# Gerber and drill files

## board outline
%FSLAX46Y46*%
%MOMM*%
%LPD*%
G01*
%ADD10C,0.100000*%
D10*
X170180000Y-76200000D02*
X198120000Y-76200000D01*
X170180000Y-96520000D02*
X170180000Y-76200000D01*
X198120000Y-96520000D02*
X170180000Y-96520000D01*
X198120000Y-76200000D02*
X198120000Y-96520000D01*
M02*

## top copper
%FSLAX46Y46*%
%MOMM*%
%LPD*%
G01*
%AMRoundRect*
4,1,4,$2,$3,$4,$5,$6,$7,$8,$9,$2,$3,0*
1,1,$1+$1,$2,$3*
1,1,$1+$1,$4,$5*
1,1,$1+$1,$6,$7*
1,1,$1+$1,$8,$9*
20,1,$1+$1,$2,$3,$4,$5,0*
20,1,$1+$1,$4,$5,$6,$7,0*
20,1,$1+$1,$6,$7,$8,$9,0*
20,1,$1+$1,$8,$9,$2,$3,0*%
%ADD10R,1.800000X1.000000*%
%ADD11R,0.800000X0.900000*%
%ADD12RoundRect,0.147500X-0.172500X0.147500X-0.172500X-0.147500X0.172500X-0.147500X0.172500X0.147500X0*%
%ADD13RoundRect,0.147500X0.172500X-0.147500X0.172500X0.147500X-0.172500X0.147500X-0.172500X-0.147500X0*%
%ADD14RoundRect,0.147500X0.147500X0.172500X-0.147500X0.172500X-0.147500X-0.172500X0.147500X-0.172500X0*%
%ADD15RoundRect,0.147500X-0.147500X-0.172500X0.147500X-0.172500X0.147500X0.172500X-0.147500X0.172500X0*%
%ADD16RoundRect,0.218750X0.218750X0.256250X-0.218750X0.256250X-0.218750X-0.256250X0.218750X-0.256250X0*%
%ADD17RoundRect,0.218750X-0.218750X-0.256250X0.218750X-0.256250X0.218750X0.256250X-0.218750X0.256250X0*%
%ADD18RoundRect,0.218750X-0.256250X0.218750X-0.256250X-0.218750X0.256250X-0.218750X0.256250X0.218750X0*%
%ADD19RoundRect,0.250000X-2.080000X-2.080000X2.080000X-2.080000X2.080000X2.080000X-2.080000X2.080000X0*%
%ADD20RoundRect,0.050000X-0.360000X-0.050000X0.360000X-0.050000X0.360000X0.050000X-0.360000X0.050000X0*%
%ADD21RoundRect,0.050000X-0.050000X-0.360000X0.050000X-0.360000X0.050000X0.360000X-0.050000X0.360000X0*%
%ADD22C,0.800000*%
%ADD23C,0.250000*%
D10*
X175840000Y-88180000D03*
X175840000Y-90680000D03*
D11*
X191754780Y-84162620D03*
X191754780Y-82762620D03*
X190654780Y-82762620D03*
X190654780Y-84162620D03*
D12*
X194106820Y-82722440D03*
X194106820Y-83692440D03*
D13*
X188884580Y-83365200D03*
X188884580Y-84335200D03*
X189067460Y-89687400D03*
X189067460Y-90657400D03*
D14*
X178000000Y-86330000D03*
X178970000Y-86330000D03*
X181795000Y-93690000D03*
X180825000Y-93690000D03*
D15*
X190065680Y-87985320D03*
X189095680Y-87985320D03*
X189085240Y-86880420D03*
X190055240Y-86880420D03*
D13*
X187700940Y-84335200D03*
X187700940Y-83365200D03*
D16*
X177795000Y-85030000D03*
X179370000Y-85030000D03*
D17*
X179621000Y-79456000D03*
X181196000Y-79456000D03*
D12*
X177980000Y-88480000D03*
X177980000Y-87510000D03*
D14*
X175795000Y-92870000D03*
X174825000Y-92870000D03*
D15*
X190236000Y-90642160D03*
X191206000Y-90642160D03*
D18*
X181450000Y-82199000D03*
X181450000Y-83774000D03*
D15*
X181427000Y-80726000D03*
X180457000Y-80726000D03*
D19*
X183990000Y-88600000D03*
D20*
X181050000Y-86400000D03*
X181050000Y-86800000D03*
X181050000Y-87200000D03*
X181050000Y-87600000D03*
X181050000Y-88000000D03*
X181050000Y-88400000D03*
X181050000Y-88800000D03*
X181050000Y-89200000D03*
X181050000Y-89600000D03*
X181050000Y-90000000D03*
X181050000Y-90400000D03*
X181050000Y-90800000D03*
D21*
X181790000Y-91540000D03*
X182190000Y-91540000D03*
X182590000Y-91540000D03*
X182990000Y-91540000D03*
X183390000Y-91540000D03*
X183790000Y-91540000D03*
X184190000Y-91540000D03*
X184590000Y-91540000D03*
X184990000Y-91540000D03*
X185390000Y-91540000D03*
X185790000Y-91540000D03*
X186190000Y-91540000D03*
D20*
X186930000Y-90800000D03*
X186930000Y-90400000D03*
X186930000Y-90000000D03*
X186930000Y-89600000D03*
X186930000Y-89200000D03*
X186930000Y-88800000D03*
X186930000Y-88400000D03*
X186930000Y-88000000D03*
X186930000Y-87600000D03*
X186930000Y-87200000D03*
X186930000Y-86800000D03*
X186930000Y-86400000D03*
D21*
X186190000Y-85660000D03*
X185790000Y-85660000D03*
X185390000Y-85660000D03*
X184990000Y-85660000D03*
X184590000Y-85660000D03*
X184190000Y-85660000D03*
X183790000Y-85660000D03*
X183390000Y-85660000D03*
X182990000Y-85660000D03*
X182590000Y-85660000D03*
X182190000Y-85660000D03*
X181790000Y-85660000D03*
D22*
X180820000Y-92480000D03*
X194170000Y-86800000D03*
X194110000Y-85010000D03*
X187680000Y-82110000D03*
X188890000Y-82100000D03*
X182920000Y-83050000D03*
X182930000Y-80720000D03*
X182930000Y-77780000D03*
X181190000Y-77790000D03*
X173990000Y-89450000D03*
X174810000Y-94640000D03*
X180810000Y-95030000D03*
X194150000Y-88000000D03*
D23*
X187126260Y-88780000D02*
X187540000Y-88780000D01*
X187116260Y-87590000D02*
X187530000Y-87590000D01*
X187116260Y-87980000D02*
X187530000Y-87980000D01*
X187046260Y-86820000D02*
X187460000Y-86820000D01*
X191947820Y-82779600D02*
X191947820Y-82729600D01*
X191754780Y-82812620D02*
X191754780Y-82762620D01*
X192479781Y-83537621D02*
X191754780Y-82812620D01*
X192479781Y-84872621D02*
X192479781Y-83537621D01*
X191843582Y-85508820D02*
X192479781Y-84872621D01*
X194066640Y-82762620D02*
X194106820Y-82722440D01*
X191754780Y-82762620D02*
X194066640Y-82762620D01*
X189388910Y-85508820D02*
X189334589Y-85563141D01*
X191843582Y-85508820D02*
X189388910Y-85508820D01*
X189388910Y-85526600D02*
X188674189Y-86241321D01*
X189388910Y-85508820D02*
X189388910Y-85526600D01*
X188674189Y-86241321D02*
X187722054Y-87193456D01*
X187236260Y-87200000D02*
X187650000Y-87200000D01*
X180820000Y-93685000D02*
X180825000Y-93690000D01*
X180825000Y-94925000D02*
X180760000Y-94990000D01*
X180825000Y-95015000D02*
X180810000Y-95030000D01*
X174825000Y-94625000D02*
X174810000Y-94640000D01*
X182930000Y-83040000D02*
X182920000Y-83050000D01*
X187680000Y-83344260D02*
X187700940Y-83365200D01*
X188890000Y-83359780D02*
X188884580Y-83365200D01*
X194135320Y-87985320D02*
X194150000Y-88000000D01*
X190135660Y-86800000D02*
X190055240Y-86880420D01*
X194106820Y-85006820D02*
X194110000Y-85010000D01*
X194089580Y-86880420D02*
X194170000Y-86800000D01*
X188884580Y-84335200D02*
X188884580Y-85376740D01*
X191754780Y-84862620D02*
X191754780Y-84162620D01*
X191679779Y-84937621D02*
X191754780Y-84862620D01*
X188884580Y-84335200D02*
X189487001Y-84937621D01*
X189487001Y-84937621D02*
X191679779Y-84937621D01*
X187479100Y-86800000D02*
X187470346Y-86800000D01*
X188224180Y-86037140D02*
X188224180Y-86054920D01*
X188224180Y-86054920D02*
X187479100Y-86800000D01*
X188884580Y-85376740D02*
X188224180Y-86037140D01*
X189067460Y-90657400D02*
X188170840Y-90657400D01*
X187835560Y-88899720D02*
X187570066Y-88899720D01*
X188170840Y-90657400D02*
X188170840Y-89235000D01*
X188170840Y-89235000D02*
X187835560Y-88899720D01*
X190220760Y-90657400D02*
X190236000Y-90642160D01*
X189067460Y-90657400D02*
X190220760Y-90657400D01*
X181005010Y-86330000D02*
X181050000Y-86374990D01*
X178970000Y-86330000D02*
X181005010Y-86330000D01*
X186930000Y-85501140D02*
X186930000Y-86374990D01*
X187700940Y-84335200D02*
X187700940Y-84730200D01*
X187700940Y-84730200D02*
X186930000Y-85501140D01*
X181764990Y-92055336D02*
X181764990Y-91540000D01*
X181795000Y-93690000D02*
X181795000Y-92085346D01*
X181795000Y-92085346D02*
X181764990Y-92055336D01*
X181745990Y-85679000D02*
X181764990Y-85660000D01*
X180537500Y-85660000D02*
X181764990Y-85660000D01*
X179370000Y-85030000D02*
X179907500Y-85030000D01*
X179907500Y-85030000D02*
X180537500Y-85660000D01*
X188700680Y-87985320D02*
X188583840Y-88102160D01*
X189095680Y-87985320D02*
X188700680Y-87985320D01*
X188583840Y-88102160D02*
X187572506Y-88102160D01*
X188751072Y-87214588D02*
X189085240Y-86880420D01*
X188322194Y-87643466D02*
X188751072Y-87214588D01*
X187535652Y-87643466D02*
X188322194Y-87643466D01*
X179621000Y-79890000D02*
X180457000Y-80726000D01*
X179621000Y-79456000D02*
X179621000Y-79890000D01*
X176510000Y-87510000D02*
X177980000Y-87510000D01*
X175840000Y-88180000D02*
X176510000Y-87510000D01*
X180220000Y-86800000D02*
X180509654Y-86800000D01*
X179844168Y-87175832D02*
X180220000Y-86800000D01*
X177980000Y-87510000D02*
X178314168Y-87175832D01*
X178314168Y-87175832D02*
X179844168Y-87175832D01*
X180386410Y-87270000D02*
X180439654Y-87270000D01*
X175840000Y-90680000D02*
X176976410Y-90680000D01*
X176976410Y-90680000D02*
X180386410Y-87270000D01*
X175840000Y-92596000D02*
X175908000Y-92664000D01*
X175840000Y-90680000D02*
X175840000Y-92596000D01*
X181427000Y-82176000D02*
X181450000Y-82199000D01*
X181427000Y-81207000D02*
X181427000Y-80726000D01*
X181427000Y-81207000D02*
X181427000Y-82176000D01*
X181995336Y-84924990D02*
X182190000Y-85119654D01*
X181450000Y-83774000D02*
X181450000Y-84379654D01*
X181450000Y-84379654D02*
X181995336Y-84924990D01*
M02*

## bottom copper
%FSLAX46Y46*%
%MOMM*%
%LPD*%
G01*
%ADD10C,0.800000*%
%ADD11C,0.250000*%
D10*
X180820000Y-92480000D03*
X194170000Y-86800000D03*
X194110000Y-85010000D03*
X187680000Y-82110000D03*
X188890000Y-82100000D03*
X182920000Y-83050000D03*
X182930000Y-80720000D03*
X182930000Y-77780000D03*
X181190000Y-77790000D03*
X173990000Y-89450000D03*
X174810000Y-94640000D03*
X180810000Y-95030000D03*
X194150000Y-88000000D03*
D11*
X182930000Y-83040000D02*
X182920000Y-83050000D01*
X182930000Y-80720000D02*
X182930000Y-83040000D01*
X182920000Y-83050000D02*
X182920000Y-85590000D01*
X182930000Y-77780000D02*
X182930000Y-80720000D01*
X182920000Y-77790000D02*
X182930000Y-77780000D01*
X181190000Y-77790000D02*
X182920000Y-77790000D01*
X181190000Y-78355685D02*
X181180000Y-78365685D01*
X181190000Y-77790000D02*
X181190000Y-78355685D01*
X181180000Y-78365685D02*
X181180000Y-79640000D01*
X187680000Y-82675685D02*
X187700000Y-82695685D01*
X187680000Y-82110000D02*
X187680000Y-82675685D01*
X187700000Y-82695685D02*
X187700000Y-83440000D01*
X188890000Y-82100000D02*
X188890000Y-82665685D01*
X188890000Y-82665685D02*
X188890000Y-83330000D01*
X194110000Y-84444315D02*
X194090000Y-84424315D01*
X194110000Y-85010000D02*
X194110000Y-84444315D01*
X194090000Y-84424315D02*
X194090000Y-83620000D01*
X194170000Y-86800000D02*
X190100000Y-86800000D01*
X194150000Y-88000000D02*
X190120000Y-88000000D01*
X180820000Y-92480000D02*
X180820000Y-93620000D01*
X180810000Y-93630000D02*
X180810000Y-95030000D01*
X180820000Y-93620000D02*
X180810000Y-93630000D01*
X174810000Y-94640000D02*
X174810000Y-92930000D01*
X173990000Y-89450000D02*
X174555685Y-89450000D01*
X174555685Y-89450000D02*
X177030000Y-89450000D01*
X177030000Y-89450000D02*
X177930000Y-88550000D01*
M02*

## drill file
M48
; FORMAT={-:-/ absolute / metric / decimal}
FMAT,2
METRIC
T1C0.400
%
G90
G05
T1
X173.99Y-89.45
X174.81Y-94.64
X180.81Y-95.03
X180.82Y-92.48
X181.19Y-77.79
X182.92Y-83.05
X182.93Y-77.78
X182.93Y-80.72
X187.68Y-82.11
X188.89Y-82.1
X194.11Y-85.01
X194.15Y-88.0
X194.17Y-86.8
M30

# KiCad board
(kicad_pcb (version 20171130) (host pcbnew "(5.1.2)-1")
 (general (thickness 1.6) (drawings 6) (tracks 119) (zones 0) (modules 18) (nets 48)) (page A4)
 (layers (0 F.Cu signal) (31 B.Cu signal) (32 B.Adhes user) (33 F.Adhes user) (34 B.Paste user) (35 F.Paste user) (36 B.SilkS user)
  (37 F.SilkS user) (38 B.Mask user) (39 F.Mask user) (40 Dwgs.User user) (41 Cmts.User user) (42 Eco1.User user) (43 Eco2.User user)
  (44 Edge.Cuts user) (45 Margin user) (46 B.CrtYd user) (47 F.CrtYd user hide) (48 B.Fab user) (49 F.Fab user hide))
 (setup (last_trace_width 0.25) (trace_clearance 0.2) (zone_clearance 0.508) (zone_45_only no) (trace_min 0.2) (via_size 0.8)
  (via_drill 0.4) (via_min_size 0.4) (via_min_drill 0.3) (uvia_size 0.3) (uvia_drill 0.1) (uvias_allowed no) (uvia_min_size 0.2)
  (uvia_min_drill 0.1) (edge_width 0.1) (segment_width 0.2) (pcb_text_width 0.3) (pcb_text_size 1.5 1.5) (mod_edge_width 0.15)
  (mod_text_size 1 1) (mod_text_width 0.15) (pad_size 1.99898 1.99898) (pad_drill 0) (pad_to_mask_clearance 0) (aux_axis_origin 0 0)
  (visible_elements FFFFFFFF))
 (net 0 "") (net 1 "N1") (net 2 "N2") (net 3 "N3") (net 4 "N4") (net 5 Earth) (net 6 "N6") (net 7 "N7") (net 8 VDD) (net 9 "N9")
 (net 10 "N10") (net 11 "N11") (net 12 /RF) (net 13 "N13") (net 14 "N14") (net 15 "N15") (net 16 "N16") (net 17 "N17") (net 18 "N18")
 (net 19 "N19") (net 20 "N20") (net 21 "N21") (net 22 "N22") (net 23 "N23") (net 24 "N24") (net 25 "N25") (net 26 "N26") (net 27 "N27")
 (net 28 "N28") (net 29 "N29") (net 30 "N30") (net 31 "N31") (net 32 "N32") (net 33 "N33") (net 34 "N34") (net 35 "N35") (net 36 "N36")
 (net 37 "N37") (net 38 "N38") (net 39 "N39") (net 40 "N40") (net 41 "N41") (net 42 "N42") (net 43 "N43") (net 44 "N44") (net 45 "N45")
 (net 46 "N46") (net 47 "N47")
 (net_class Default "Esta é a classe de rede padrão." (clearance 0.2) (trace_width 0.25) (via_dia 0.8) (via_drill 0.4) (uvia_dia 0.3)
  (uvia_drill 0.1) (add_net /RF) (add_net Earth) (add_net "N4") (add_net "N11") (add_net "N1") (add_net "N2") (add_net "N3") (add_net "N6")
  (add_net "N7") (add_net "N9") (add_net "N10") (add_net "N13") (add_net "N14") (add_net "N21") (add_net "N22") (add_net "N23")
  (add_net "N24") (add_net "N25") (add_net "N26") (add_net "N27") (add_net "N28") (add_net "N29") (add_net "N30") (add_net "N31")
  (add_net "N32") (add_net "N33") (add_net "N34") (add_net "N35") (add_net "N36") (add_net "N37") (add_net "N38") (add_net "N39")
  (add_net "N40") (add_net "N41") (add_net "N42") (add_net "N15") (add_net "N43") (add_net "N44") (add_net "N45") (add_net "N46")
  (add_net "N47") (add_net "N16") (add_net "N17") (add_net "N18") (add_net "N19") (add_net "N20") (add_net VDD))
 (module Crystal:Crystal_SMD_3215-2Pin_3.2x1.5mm (layer F.Cu) (at 175.84 89.43 90)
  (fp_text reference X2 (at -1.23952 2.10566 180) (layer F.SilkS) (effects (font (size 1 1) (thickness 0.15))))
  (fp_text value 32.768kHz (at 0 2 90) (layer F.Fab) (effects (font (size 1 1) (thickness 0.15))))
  (pad 1 smd rect (at 1.25 0 90) (size 1 1.8) (layers F.Cu F.Paste F.Mask) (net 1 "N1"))
  (pad 2 smd rect (at -1.25 0 90) (size 1 1.8) (layers F.Cu F.Paste F.Mask) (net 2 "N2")))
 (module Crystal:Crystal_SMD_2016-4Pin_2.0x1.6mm (layer F.Cu) (at 191.20478 83.46262 90)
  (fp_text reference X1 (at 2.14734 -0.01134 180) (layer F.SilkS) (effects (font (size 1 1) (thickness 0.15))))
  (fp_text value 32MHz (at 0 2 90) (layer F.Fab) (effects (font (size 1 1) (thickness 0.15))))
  (pad 1 smd rect (at -0.7 0.55 90) (size 0.9 0.8) (layers F.Cu F.Paste F.Mask) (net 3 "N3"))
  (pad 2 smd rect (at 0.7 0.55 90) (size 0.9 0.8) (layers F.Cu F.Paste F.Mask) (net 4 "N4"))
  (pad 3 smd rect (at 0.7 -0.55 90) (size 0.9 0.8) (layers F.Cu F.Paste F.Mask))
  (pad 4 smd rect (at -0.7 -0.55 90) (size 0.9 0.8) (layers F.Cu F.Paste F.Mask)))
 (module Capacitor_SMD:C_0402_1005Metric (layer F.Cu) (at 194.10682 83.20744 270)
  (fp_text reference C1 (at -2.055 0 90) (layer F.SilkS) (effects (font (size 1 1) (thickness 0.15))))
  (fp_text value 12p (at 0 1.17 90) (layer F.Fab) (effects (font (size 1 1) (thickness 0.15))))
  (pad 1 smd roundrect (at -0.485 0 270) (size 0.59 0.64) (layers F.Cu F.Paste F.Mask) (roundrect_rratio 0.25) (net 4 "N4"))
  (pad 2 smd roundrect (at 0.485 0 270) (size 0.59 0.64) (layers F.Cu F.Paste F.Mask) (roundrect_rratio 0.25) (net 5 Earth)))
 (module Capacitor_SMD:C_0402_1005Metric (layer F.Cu) (at 188.88458 83.8502 90)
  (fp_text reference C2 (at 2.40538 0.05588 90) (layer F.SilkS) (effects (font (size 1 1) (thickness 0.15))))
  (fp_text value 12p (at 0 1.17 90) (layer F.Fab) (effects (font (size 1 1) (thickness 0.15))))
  (pad 2 smd roundrect (at 0.485 0 90) (size 0.59 0.64) (layers F.Cu F.Paste F.Mask) (roundrect_rratio 0.25) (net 5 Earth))
  (pad 1 smd roundrect (at -0.485 0 90) (size 0.59 0.64) (layers F.Cu F.Paste F.Mask) (roundrect_rratio 0.25) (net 3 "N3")))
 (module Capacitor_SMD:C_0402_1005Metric (layer F.Cu) (at 189.06746 90.1724 90)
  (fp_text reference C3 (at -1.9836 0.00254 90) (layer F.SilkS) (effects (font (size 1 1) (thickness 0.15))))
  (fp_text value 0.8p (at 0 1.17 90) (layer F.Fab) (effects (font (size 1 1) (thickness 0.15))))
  (pad 2 smd roundrect (at 0.485 0 90) (size 0.59 0.64) (layers F.Cu F.Paste F.Mask) (roundrect_rratio 0.25) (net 5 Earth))
  (pad 1 smd roundrect (at -0.485 0 90) (size 0.59 0.64) (layers F.Cu F.Paste F.Mask) (roundrect_rratio 0.25) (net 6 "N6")))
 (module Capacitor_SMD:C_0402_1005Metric (layer F.Cu) (at 178.485 86.33 180)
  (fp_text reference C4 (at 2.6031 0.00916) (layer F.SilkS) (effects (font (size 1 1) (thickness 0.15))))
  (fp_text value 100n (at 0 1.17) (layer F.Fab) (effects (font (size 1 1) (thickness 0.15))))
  (pad 2 smd roundrect (at 0.485 0 180) (size 0.59 0.64) (layers F.Cu F.Paste F.Mask) (roundrect_rratio 0.25) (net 5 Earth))
  (pad 1 smd roundrect (at -0.485 0 180) (size 0.59 0.64) (layers F.Cu F.Paste F.Mask) (roundrect_rratio 0.25) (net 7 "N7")))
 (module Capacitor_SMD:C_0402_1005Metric (layer F.Cu) (at 181.31 93.69 180)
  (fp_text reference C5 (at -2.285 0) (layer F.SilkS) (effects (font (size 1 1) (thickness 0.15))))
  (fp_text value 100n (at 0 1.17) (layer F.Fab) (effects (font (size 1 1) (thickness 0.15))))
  (pad 1 smd roundrect (at -0.485 0 180) (size 0.59 0.64) (layers F.Cu F.Paste F.Mask) (roundrect_rratio 0.25) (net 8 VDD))
  (pad 2 smd roundrect (at 0.485 0 180) (size 0.59 0.64) (layers F.Cu F.Paste F.Mask) (roundrect_rratio 0.25) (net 5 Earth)))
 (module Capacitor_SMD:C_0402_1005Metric (layer F.Cu) (at 189.58068 87.98532)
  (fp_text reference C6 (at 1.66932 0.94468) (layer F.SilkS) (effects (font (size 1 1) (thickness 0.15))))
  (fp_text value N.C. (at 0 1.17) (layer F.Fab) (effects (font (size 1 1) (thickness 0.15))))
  (pad 2 smd roundrect (at 0.485 0) (size 0.59 0.64) (layers F.Cu F.Paste F.Mask) (roundrect_rratio 0.25) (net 5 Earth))
  (pad 1 smd roundrect (at -0.485 0) (size 0.59 0.64) (layers F.Cu F.Paste F.Mask) (roundrect_rratio 0.25) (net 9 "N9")))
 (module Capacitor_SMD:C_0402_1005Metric (layer F.Cu) (at 189.57024 86.88042)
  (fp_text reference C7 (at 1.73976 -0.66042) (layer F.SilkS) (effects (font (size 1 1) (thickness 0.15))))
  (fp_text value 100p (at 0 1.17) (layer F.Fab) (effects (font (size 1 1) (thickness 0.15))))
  (pad 1 smd roundrect (at -0.485 0) (size 0.59 0.64) (layers F.Cu F.Paste F.Mask) (roundrect_rratio 0.25) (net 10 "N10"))
  (pad 2 smd roundrect (at 0.485 0) (size 0.59 0.64) (layers F.Cu F.Paste F.Mask) (roundrect_rratio 0.25) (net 5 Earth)))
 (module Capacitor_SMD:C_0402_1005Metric (layer F.Cu) (at 187.70094 83.8502 90)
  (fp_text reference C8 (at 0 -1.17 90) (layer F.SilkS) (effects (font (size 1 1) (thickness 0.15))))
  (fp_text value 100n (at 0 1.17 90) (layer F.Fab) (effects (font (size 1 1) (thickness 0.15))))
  (pad 1 smd roundrect (at -0.485 0 90) (size 0.59 0.64) (layers F.Cu F.Paste F.Mask) (roundrect_rratio 0.25) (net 8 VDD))
  (pad 2 smd roundrect (at 0.485 0 90) (size 0.59 0.64) (layers F.Cu F.Paste F.Mask) (roundrect_rratio 0.25) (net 5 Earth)))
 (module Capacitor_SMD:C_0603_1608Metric (layer F.Cu) (at 178.5825 85.03 180)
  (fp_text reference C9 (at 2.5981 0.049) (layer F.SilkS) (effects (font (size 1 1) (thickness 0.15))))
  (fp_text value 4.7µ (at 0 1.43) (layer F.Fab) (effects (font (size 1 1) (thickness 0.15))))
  (pad 2 smd roundrect (at 0.7875 0 180) (size 0.875 0.95) (layers F.Cu F.Paste F.Mask) (roundrect_rratio 0.25) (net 5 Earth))
  (pad 1 smd roundrect (at -0.7875 0 180) (size 0.875 0.95) (layers F.Cu F.Paste F.Mask) (roundrect_rratio 0.25) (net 8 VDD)))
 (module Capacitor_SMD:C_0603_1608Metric (layer F.Cu) (at 180.4085 79.456)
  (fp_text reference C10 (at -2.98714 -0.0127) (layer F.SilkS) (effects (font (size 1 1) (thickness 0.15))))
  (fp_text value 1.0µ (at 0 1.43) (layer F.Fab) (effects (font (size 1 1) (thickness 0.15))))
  (pad 1 smd roundrect (at -0.7875 0) (size 0.875 0.95) (layers F.Cu F.Paste F.Mask) (roundrect_rratio 0.25) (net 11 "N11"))
  (pad 2 smd roundrect (at 0.7875 0) (size 0.875 0.95) (layers F.Cu F.Paste F.Mask) (roundrect_rratio 0.25) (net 5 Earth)))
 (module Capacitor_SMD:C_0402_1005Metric (layer F.Cu) (at 177.98 87.995 270)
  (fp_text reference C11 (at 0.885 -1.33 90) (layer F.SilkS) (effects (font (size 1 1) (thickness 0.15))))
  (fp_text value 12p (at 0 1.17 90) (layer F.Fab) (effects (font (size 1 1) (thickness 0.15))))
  (pad 2 smd roundrect (at 0.485 0 270) (size 0.59 0.64) (layers F.Cu F.Paste F.Mask) (roundrect_rratio 0.25) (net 5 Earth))
  (pad 1 smd roundrect (at -0.485 0 270) (size 0.59 0.64) (layers F.Cu F.Paste F.Mask) (roundrect_rratio 0.25) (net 1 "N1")))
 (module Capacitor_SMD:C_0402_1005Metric (layer F.Cu) (at 175.31 92.87 180)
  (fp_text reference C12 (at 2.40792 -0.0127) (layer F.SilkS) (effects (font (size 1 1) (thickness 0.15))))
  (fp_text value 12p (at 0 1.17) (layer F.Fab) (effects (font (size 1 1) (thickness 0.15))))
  (pad 1 smd roundrect (at -0.485 0 180) (size 0.59 0.64) (layers F.Cu F.Paste F.Mask) (roundrect_rratio 0.25) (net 2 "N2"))
  (pad 2 smd roundrect (at 0.485 0 180) (size 0.59 0.64) (layers F.Cu F.Paste F.Mask) (roundrect_rratio 0.25) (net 5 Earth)))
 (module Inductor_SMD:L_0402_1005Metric (layer F.Cu) (at 190.721 90.64216)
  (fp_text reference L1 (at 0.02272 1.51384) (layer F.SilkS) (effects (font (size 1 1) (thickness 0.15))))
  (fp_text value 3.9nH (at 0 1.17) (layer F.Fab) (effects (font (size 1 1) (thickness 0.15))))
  (pad 1 smd roundrect (at -0.485 0) (size 0.59 0.64) (layers F.Cu F.Paste F.Mask) (roundrect_rratio 0.25) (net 6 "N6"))
  (pad 2 smd roundrect (at 0.485 0) (size 0.59 0.64) (layers F.Cu F.Paste F.Mask) (roundrect_rratio 0.25) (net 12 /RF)))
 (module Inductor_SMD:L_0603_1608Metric (layer F.Cu) (at 181.45 82.9865 270)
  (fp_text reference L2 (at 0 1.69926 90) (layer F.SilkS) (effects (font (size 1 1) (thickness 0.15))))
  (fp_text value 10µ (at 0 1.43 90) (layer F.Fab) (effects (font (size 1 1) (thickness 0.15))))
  (pad 1 smd roundrect (at -0.7875 0 270) (size 0.875 0.95) (layers F.Cu F.Paste F.Mask) (roundrect_rratio 0.25) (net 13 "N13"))
  (pad 2 smd roundrect (at 0.7875 0 270) (size 0.875 0.95) (layers F.Cu F.Paste F.Mask) (roundrect_rratio 0.25) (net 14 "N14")))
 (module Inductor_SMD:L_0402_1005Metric (layer F.Cu) (at 180.942 80.726)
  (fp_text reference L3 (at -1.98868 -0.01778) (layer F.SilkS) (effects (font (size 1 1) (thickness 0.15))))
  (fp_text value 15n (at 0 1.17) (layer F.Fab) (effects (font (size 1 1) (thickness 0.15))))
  (pad 2 smd roundrect (at 0.485 0) (size 0.59 0.64) (layers F.Cu F.Paste F.Mask) (roundrect_rratio 0.25) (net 13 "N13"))
  (pad 1 smd roundrect (at -0.485 0) (size 0.59 0.64) (layers F.Cu F.Paste F.Mask) (roundrect_rratio 0.25) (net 11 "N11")))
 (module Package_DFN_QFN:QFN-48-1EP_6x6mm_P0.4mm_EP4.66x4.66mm (layer F.Cu) (at 183.99 88.6)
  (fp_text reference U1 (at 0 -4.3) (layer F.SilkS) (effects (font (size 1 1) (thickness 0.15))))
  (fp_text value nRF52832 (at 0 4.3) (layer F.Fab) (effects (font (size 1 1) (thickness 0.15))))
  (pad 49 smd roundrect (at 0 0) (size 4.66 4.66) (layers F.Cu F.Mask) (roundrect_rratio 0.053648))
  (pad "" smd roundrect (at -1.55 -1.55) (size 1.25 1.25) (layers F.Paste) (roundrect_rratio 0.2))
  (pad "" smd roundrect (at -1.55 0) (size 1.25 1.25) (layers F.Paste) (roundrect_rratio 0.2))
  (pad "" smd roundrect (at -1.55 1.55) (size 1.25 1.25) (layers F.Paste) (roundrect_rratio 0.2))
  (pad "" smd roundrect (at 0 -1.55) (size 1.25 1.25) (layers F.Paste) (roundrect_rratio 0.2))
  (pad "" smd roundrect (at 0 0) (size 1.25 1.25) (layers F.Paste) (roundrect_rratio 0.2))
  (pad "" smd roundrect (at 0 1.55) (size 1.25 1.25) (layers F.Paste) (roundrect_rratio 0.2))
  (pad "" smd roundrect (at 1.55 -1.55) (size 1.25 1.25) (layers F.Paste) (roundrect_rratio 0.2))
  (pad "" smd roundrect (at 1.55 0) (size 1.25 1.25) (layers F.Paste) (roundrect_rratio 0.2))
  (pad "" smd roundrect (at 1.55 1.55) (size 1.25 1.25) (layers F.Paste) (roundrect_rratio 0.2))
  (pad 1 smd roundrect (at -2.94 -2.2) (size 0.82 0.2) (layers F.Cu F.Paste F.Mask) (roundrect_rratio 0.25) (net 7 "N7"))
  (pad 2 smd roundrect (at -2.94 -1.8) (size 0.82 0.2) (layers F.Cu F.Paste F.Mask) (roundrect_rratio 0.25) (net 1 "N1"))
  (pad 3 smd roundrect (at -2.94 -1.4) (size 0.82 0.2) (layers F.Cu F.Paste F.Mask) (roundrect_rratio 0.25) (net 2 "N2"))
  (pad 4 smd roundrect (at -2.94 -1) (size 0.82 0.2) (layers F.Cu F.Paste F.Mask) (roundrect_rratio 0.25) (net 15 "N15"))
  (pad 5 smd roundrect (at -2.94 -0.6) (size 0.82 0.2) (layers F.Cu F.Paste F.Mask) (roundrect_rratio 0.25) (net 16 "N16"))
  (pad 6 smd roundrect (at -2.94 -0.2) (size 0.82 0.2) (layers F.Cu F.Paste F.Mask) (roundrect_rratio 0.25) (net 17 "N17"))
  (pad 7 smd roundrect (at -2.94 0.2) (size 0.82 0.2) (layers F.Cu F.Paste F.Mask) (roundrect_rratio 0.25) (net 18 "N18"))
  (pad 8 smd roundrect (at -2.94 0.6) (size 0.82 0.2) (layers F.Cu F.Paste F.Mask) (roundrect_rratio 0.25) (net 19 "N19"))
  (pad 9 smd roundrect (at -2.94 1) (size 0.82 0.2) (layers F.Cu F.Paste F.Mask) (roundrect_rratio 0.25) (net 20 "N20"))
  (pad 10 smd roundrect (at -2.94 1.4) (size 0.82 0.2) (layers F.Cu F.Paste F.Mask) (roundrect_rratio 0.25) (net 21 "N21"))
  (pad 11 smd roundrect (at -2.94 1.8) (size 0.82 0.2) (layers F.Cu F.Paste F.Mask) (roundrect_rratio 0.25) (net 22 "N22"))
  (pad 12 smd roundrect (at -2.94 2.2) (size 0.82 0.2) (layers F.Cu F.Paste F.Mask) (roundrect_rratio 0.25) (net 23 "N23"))
  (pad 13 smd roundrect (at -2.2 2.94) (size 0.2 0.82) (layers F.Cu F.Paste F.Mask) (roundrect_rratio 0.25) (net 8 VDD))
  (pad 14 smd roundrect (at -1.8 2.94) (size 0.2 0.82) (layers F.Cu F.Paste F.Mask) (roundrect_rratio 0.25) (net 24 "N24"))
  (pad 15 smd roundrect (at -1.4 2.94) (size 0.2 0.82) (layers F.Cu F.Paste F.Mask) (roundrect_rratio 0.25) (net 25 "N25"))
  (pad 16 smd roundrect (at -1 2.94) (size 0.2 0.82) (layers F.Cu F.Paste F.Mask) (roundrect_rratio 0.25) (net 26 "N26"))
  (pad 17 smd roundrect (at -0.6 2.94) (size 0.2 0.82) (layers F.Cu F.Paste F.Mask) (roundrect_rratio 0.25) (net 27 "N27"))
  (pad 18 smd roundrect (at -0.2 2.94) (size 0.2 0.82) (layers F.Cu F.Paste F.Mask) (roundrect_rratio 0.25) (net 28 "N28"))
  (pad 19 smd roundrect (at 0.2 2.94) (size 0.2 0.82) (layers F.Cu F.Paste F.Mask) (roundrect_rratio 0.25) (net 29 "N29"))
  (pad 20 smd roundrect (at 0.6 2.94) (size 0.2 0.82) (layers F.Cu F.Paste F.Mask) (roundrect_rratio 0.25) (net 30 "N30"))
  (pad 21 smd roundrect (at 1 2.94) (size 0.2 0.82) (layers F.Cu F.Paste F.Mask) (roundrect_rratio 0.25) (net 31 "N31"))
  (pad 22 smd roundrect (at 1.4 2.94) (size 0.2 0.82) (layers F.Cu F.Paste F.Mask) (roundrect_rratio 0.25) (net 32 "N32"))
  (pad 23 smd roundrect (at 1.8 2.94) (size 0.2 0.82) (layers F.Cu F.Paste F.Mask) (roundrect_rratio 0.25) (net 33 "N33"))
  (pad 24 smd roundrect (at 2.2 2.94) (size 0.2 0.82) (layers F.Cu F.Paste F.Mask) (roundrect_rratio 0.25) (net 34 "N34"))
  (pad 25 smd roundrect (at 2.94 2.2) (size 0.82 0.2) (layers F.Cu F.Paste F.Mask) (roundrect_rratio 0.25) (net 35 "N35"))
  (pad 26 smd roundrect (at 2.94 1.8) (size 0.82 0.2) (layers F.Cu F.Paste F.Mask) (roundrect_rratio 0.25) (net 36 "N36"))
  (pad 27 smd roundrect (at 2.94 1.4) (size 0.82 0.2) (layers F.Cu F.Paste F.Mask) (roundrect_rratio 0.25) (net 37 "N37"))
  (pad 28 smd roundrect (at 2.94 1) (size 0.82 0.2) (layers F.Cu F.Paste F.Mask) (roundrect_rratio 0.25) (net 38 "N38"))
  (pad 29 smd roundrect (at 2.94 0.6) (size 0.82 0.2) (layers F.Cu F.Paste F.Mask) (roundrect_rratio 0.25) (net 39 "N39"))
  (pad 30 smd roundrect (at 2.94 0.2) (size 0.82 0.2) (layers F.Cu F.Paste F.Mask) (roundrect_rratio 0.25) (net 6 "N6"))
  (pad 31 smd roundrect (at 2.94 -0.2) (size 0.82 0.2) (layers F.Cu F.Paste F.Mask) (roundrect_rratio 0.25) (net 5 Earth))
  (pad 32 smd roundrect (at 2.94 -0.6) (size 0.82 0.2) (layers F.Cu F.Paste F.Mask) (roundrect_rratio 0.25) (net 9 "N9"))
  (pad 33 smd roundrect (at 2.94 -1) (size 0.82 0.2) (layers F.Cu F.Paste F.Mask) (roundrect_rratio 0.25) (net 10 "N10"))
  (pad 34 smd roundrect (at 2.94 -1.4) (size 0.82 0.2) (layers F.Cu F.Paste F.Mask) (roundrect_rratio 0.25) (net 4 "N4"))
  (pad 35 smd roundrect (at 2.94 -1.8) (size 0.82 0.2) (layers F.Cu F.Paste F.Mask) (roundrect_rratio 0.25) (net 3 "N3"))
  (pad 36 smd roundrect (at 2.94 -2.2) (size 0.82 0.2) (layers F.Cu F.Paste F.Mask) (roundrect_rratio 0.25) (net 8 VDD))
  (pad 37 smd roundrect (at 2.2 -2.94) (size 0.2 0.82) (layers F.Cu F.Paste F.Mask) (roundrect_rratio 0.25) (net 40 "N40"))
  (pad 38 smd roundrect (at 1.8 -2.94) (size 0.2 0.82) (layers F.Cu F.Paste F.Mask) (roundrect_rratio 0.25) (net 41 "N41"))
  (pad 39 smd roundrect (at 1.4 -2.94) (size 0.2 0.82) (layers F.Cu F.Paste F.Mask) (roundrect_rratio 0.25) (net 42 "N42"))
  (pad 40 smd roundrect (at 1 -2.94) (size 0.2 0.82) (layers F.Cu F.Paste F.Mask) (roundrect_rratio 0.25) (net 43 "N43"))
  (pad 41 smd roundrect (at 0.6 -2.94) (size 0.2 0.82) (layers F.Cu F.Paste F.Mask) (roundrect_rratio 0.25) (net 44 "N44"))
  (pad 42 smd roundrect (at 0.2 -2.94) (size 0.2 0.82) (layers F.Cu F.Paste F.Mask) (roundrect_rratio 0.25) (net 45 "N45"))
  (pad 43 smd roundrect (at -0.2 -2.94) (size 0.2 0.82) (layers F.Cu F.Paste F.Mask) (roundrect_rratio 0.25) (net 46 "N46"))
  (pad 44 smd roundrect (at -0.6 -2.94) (size 0.2 0.82) (layers F.Cu F.Paste F.Mask) (roundrect_rratio 0.25) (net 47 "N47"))
  (pad 45 smd roundrect (at -1 -2.94) (size 0.2 0.82) (layers F.Cu F.Paste F.Mask) (roundrect_rratio 0.25) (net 5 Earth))
  (pad 46 smd roundrect (at -1.4 -2.94) (size 0.2 0.82) (layers F.Cu F.Paste F.Mask) (roundrect_rratio 0.25) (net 11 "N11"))
  (pad 47 smd roundrect (at -1.8 -2.94) (size 0.2 0.82) (layers F.Cu F.Paste F.Mask) (roundrect_rratio 0.25) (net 14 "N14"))
  (pad 48 smd roundrect (at -2.2 -2.94) (size 0.2 0.82) (layers F.Cu F.Paste F.Mask) (roundrect_rratio 0.25) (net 8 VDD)))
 (gr_line (start 170.18 76.2) (end 198.12 76.2) (layer Edge.Cuts) (width 0.1))
 (gr_line (start 170.18 96.52) (end 170.18 76.2) (layer Edge.Cuts) (width 0.1))
 (gr_line (start 198.12 96.52) (end 170.18 96.52) (layer Edge.Cuts) (width 0.1))
 (gr_line (start 198.12 76.2) (end 198.12 96.52) (layer Edge.Cuts) (width 0.1))
 (segment (start 187.12626 88.78) (end 187.54 88.78) (width 0.25) (layer F.Cu) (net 6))
 (segment (start 187.11626 87.59) (end 187.53 87.59) (width 0.25) (layer F.Cu) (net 10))
 (segment (start 187.11626 87.98) (end 187.53 87.98) (width 0.25) (layer F.Cu) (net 9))
 (segment (start 187.04626 86.82) (end 187.46 86.82) (width 0.25) (layer F.Cu) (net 3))
 (via (at 180.82 92.48) (size 0.8) (drill 0.4) (layers F.Cu B.Cu) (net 5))
 (via (at 194.17 86.8) (size 0.8) (drill 0.4) (layers F.Cu B.Cu) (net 5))
 (via (at 194.11 85.01) (size 0.8) (drill 0.4) (layers F.Cu B.Cu) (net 5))
 (via (at 187.68 82.11) (size 0.8) (drill 0.4) (layers F.Cu B.Cu) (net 5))
 (via (at 188.89 82.1) (size 0.8) (drill 0.4) (layers F.Cu B.Cu) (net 5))
 (via (at 182.92 83.05) (size 0.8) (drill 0.4) (layers F.Cu B.Cu) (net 5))
 (via (at 182.93 80.72) (size 0.8) (drill 0.4) (layers F.Cu B.Cu) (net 5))
 (via (at 182.93 77.78) (size 0.8) (drill 0.4) (layers F.Cu B.Cu) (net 5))
 (via (at 181.19 77.79) (size 0.8) (drill 0.4) (layers F.Cu B.Cu) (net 5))
 (via (at 173.99 89.45) (size 0.8) (drill 0.4) (layers F.Cu B.Cu) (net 5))
 (via (at 174.81 94.64) (size 0.8) (drill 0.4) (layers F.Cu B.Cu) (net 5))
 (via (at 180.81 95.03) (size 0.8) (drill 0.4) (layers F.Cu B.Cu) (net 5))
 (segment (start 191.94782 82.7796) (end 191.94782 82.7296) (width 0.25) (layer F.Cu) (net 4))
 (segment (start 191.75478 82.81262) (end 191.75478 82.76262) (width 0.25) (layer F.Cu) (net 4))
 (segment (start 192.479781 83.537621) (end 191.75478 82.81262) (width 0.25) (layer F.Cu) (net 4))
 (segment (start 192.479781 84.872621) (end 192.479781 83.537621) (width 0.25) (layer F.Cu) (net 4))
 (segment (start 191.843582 85.50882) (end 192.479781 84.872621) (width 0.25) (layer F.Cu) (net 4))
 (segment (start 194.06664 82.76262) (end 194.10682 82.72244) (width 0.25) (layer F.Cu) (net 4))
 (segment (start 191.75478 82.76262) (end 194.06664 82.76262) (width 0.25) (layer F.Cu) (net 4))
 (segment (start 189.38891 85.50882) (end 189.334589 85.563141) (width 0.25) (layer F.Cu) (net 4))
 (segment (start 191.843582 85.50882) (end 189.38891 85.50882) (width 0.25) (layer F.Cu) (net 4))
 (segment (start 189.38891 85.5266) (end 188.674189 86.241321) (width 0.25) (layer F.Cu) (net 4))
 (segment (start 189.38891 85.50882) (end 189.38891 85.5266) (width 0.25) (layer F.Cu) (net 4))
 (segment (start 188.674189 86.241321) (end 187.722054 87.193456) (width 0.25) (layer F.Cu) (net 4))
 (segment (start 187.23626 87.2) (end 187.65 87.2) (width 0.25) (layer F.Cu) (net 4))
 (segment (start 180.82 93.685) (end 180.825 93.69) (width 0.25) (layer F.Cu) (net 5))
 (segment (start 180.825 94.925) (end 180.76 94.99) (width 0.25) (layer F.Cu) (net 5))
 (segment (start 180.825 95.015) (end 180.81 95.03) (width 0.25) (layer F.Cu) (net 5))
 (segment (start 174.825 94.625) (end 174.81 94.64) (width 0.25) (layer F.Cu) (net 5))
 (segment (start 182.93 83.04) (end 182.92 83.05) (width 0.25) (layer F.Cu) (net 5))
 (segment (start 187.68 83.34426) (end 187.70094 83.3652) (width 0.25) (layer F.Cu) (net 5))
 (segment (start 188.89 83.35978) (end 188.88458 83.3652) (width 0.25) (layer F.Cu) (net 5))
 (via (at 194.15 88) (size 0.8) (drill 0.4) (layers F.Cu B.Cu) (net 5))
 (segment (start 194.13532 87.98532) (end 194.15 88) (width 0.25) (layer F.Cu) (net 5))
 (segment (start 190.13566 86.8) (end 190.05524 86.88042) (width 0.25) (layer F.Cu) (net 5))
 (segment (start 182.93 83.04) (end 182.92 83.05) (width 0.25) (layer B.Cu) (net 5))
 (segment (start 182.93 80.72) (end 182.93 83.04) (width 0.25) (layer B.Cu) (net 5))
 (segment (start 182.92 83.05) (end 182.92 85.59) (width 0.25) (layer B.Cu) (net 5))
 (segment (start 182.93 77.78) (end 182.93 80.72) (width 0.25) (layer B.Cu) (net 5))
 (segment (start 182.92 77.79) (end 182.93 77.78) (width 0.25) (layer B.Cu) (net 5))
 (segment (start 181.19 77.79) (end 182.92 77.79) (width 0.25) (layer B.Cu) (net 5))
 (segment (start 181.19 78.355685) (end 181.18 78.365685) (width 0.25) (layer B.Cu) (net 5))
 (segment (start 181.19 77.79) (end 181.19 78.355685) (width 0.25) (layer B.Cu) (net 5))
 (segment (start 181.18 78.365685) (end 181.18 79.64) (width 0.25) (layer B.Cu) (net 5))
 (segment (start 187.68 82.675685) (end 187.7 82.695685) (width 0.25) (layer B.Cu) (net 5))
 (segment (start 187.68 82.11) (end 187.68 82.675685) (width 0.25) (layer B.Cu) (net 5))
 (segment (start 187.7 82.695685) (end 187.7 83.44) (width 0.25) (layer B.Cu) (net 5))
 (segment (start 188.89 82.1) (end 188.89 82.665685) (width 0.25) (layer B.Cu) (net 5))
 (segment (start 188.89 82.665685) (end 188.89 83.33) (width 0.25) (layer B.Cu) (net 5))
 (segment (start 194.10682 85.00682) (end 194.11 85.01) (width 0.25) (layer F.Cu) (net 5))
 (segment (start 194.11 84.444315) (end 194.09 84.424315) (width 0.25) (layer B.Cu) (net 5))
 (segment (start 194.11 85.01) (end 194.11 84.444315) (width 0.25) (layer B.Cu) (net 5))
 (segment (start 194.09 84.424315) (end 194.09 83.62) (width 0.25) (layer B.Cu) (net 5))
 (segment (start 194.08958 86.88042) (end 194.17 86.8) (width 0.25) (layer F.Cu) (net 5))
 (segment (start 194.17 86.8) (end 190.1 86.8) (width 0.25) (layer B.Cu) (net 5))
 (segment (start 194.15 88) (end 190.12 88) (width 0.25) (layer B.Cu) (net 5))
 (segment (start 180.82 92.48) (end 180.82 93.62) (width 0.25) (layer B.Cu) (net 5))
 (segment (start 180.81 93.63) (end 180.81 95.03) (width 0.25) (layer B.Cu) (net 5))
 (segment (start 180.82 93.62) (end 180.81 93.63) (width 0.25) (layer B.Cu) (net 5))
 (segment (start 174.81 94.64) (end 174.81 92.93) (width 0.25) (layer B.Cu) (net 5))
 (segment (start 173.99 89.45) (end 174.555685 89.45) (width 0.25) (layer B.Cu) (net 5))
 (segment (start 174.555685 89.45) (end 177.03 89.45) (width 0.25) (layer B.Cu) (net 5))
 (segment (start 177.03 89.45) (end 177.93 88.55) (width 0.25) (layer B.Cu) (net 5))
 (segment (start 188.88458 84.3352) (end 188.88458 85.37674) (width 0.25) (layer F.Cu) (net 3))
 (segment (start 191.75478 84.86262) (end 191.75478 84.16262) (width 0.25) (layer F.Cu) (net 3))
 (segment (start 191.679779 84.937621) (end 191.75478 84.86262) (width 0.25) (layer F.Cu) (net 3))
 (segment (start 188.88458 84.3352) (end 189.487001 84.937621) (width 0.25) (layer F.Cu) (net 3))
 (segment (start 189.487001 84.937621) (end 191.679779 84.937621) (width 0.25) (layer F.Cu) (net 3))
 (segment (start 187.4791 86.8) (end 187.470346 86.8) (width 0.25) (layer F.Cu) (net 3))
 (segment (start 188.22418 86.03714) (end 188.22418 86.05492) (width 0.25) (layer F.Cu) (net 3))
 (segment (start 188.22418 86.05492) (end 187.4791 86.8) (width 0.25) (layer F.Cu) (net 3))
 (segment (start 188.88458 85.37674) (end 188.22418 86.03714) (width 0.25) (layer F.Cu) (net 3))
 (segment (start 189.06746 90.6574) (end 188.17084 90.6574) (width 0.25) (layer F.Cu) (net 6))
 (segment (start 187.83556 88.89972) (end 187.570066 88.89972) (width 0.25) (layer F.Cu) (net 6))
 (segment (start 188.17084 90.6574) (end 188.17084 89.235) (width 0.25) (layer F.Cu) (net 6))
 (segment (start 188.17084 89.235) (end 187.83556 88.89972) (width 0.25) (layer F.Cu) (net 6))
 (segment (start 190.22076 90.6574) (end 190.236 90.64216) (width 0.25) (layer F.Cu) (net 6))
 (segment (start 189.06746 90.6574) (end 190.22076 90.6574) (width 0.25) (layer F.Cu) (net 6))
 (segment (start 181.00501 86.33) (end 181.05 86.37499) (width 0.25) (layer F.Cu) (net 7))
 (segment (start 178.97 86.33) (end 181.00501 86.33) (width 0.25) (layer F.Cu) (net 7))
 (segment (start 186.93 85.50114) (end 186.93 86.37499) (width 0.25) (layer F.Cu) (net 8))
 (segment (start 187.70094 84.3352) (end 187.70094 84.7302) (width 0.25) (layer F.Cu) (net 8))
 (segment (start 187.70094 84.7302) (end 186.93 85.50114) (width 0.25) (layer F.Cu) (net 8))
 (segment (start 181.76499 92.055336) (end 181.76499 91.54) (width 0.25) (layer F.Cu) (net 8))
 (segment (start 181.795 93.69) (end 181.795 92.085346) (width 0.25) (layer F.Cu) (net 8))
 (segment (start 181.795 92.085346) (end 181.76499 92.055336) (width 0.25) (layer F.Cu) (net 8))
 (segment (start 181.74599 85.679) (end 181.76499 85.66) (width 0.25) (layer F.Cu) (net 8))
 (segment (start 180.5375 85.66) (end 181.76499 85.66) (width 0.25) (layer F.Cu) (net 8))
 (segment (start 179.37 85.03) (end 179.9075 85.03) (width 0.25) (layer F.Cu) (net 8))
 (segment (start 179.9075 85.03) (end 180.5375 85.66) (width 0.25) (layer F.Cu) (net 8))
 (segment (start 188.70068 87.98532) (end 188.58384 88.10216) (width 0.25) (layer F.Cu) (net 9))
 (segment (start 189.09568 87.98532) (end 188.70068 87.98532) (width 0.25) (layer F.Cu) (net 9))
 (segment (start 188.58384 88.10216) (end 187.572506 88.10216) (width 0.25) (layer F.Cu) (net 9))
 (segment (start 188.751072 87.214588) (end 189.08524 86.88042) (width 0.25) (layer F.Cu) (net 10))
 (segment (start 188.322194 87.643466) (end 188.751072 87.214588) (width 0.25) (layer F.Cu) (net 10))
 (segment (start 187.535652 87.643466) (end 188.322194 87.643466) (width 0.25) (layer F.Cu) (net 10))
 (segment (start 179.621 79.89) (end 180.457 80.726) (width 0.25) (layer F.Cu) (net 11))
 (segment (start 179.621 79.456) (end 179.621 79.89) (width 0.25) (layer F.Cu) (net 11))
 (segment (start 176.51 87.51) (end 177.98 87.51) (width 0.25) (layer F.Cu) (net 1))
 (segment (start 175.84 88.18) (end 176.51 87.51) (width 0.25) (layer F.Cu) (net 1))
 (segment (start 180.22 86.8) (end 180.509654 86.8) (width 0.25) (layer F.Cu) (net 1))
 (segment (start 179.844168 87.175832) (end 180.22 86.8) (width 0.25) (layer F.Cu) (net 1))
 (segment (start 177.98 87.51) (end 178.314168 87.175832) (width 0.25) (layer F.Cu) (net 1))
 (segment (start 178.314168 87.175832) (end 179.844168 87.175832) (width 0.25) (layer F.Cu) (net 1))
 (segment (start 180.38641 87.27) (end 180.439654 87.27) (width 0.25) (layer F.Cu) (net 2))
 (segment (start 175.84 90.68) (end 176.97641 90.68) (width 0.25) (layer F.Cu) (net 2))
 (segment (start 176.97641 90.68) (end 180.38641 87.27) (width 0.25) (layer F.Cu) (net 2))
 (segment (start 175.84 92.596) (end 175.908 92.664) (width 0.25) (layer F.Cu) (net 2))
 (segment (start 175.84 90.68) (end 175.84 92.596) (width 0.25) (layer F.Cu) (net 2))
 (segment (start 181.427 82.176) (end 181.45 82.199) (width 0.25) (layer F.Cu) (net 13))
 (segment (start 181.427 81.207) (end 181.427 80.726) (width 0.25) (layer F.Cu) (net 13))
 (segment (start 181.427 81.207) (end 181.427 82.176) (width 0.25) (layer F.Cu) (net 13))
 (segment (start 181.995336 84.92499) (end 182.19 85.119654) (width 0.25) (layer F.Cu) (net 14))
 (segment (start 181.45 83.774) (end 181.45 84.379654) (width 0.25) (layer F.Cu) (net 14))
 (segment (start 181.45 84.379654) (end 181.995336 84.92499) (width 0.25) (layer F.Cu) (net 14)))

